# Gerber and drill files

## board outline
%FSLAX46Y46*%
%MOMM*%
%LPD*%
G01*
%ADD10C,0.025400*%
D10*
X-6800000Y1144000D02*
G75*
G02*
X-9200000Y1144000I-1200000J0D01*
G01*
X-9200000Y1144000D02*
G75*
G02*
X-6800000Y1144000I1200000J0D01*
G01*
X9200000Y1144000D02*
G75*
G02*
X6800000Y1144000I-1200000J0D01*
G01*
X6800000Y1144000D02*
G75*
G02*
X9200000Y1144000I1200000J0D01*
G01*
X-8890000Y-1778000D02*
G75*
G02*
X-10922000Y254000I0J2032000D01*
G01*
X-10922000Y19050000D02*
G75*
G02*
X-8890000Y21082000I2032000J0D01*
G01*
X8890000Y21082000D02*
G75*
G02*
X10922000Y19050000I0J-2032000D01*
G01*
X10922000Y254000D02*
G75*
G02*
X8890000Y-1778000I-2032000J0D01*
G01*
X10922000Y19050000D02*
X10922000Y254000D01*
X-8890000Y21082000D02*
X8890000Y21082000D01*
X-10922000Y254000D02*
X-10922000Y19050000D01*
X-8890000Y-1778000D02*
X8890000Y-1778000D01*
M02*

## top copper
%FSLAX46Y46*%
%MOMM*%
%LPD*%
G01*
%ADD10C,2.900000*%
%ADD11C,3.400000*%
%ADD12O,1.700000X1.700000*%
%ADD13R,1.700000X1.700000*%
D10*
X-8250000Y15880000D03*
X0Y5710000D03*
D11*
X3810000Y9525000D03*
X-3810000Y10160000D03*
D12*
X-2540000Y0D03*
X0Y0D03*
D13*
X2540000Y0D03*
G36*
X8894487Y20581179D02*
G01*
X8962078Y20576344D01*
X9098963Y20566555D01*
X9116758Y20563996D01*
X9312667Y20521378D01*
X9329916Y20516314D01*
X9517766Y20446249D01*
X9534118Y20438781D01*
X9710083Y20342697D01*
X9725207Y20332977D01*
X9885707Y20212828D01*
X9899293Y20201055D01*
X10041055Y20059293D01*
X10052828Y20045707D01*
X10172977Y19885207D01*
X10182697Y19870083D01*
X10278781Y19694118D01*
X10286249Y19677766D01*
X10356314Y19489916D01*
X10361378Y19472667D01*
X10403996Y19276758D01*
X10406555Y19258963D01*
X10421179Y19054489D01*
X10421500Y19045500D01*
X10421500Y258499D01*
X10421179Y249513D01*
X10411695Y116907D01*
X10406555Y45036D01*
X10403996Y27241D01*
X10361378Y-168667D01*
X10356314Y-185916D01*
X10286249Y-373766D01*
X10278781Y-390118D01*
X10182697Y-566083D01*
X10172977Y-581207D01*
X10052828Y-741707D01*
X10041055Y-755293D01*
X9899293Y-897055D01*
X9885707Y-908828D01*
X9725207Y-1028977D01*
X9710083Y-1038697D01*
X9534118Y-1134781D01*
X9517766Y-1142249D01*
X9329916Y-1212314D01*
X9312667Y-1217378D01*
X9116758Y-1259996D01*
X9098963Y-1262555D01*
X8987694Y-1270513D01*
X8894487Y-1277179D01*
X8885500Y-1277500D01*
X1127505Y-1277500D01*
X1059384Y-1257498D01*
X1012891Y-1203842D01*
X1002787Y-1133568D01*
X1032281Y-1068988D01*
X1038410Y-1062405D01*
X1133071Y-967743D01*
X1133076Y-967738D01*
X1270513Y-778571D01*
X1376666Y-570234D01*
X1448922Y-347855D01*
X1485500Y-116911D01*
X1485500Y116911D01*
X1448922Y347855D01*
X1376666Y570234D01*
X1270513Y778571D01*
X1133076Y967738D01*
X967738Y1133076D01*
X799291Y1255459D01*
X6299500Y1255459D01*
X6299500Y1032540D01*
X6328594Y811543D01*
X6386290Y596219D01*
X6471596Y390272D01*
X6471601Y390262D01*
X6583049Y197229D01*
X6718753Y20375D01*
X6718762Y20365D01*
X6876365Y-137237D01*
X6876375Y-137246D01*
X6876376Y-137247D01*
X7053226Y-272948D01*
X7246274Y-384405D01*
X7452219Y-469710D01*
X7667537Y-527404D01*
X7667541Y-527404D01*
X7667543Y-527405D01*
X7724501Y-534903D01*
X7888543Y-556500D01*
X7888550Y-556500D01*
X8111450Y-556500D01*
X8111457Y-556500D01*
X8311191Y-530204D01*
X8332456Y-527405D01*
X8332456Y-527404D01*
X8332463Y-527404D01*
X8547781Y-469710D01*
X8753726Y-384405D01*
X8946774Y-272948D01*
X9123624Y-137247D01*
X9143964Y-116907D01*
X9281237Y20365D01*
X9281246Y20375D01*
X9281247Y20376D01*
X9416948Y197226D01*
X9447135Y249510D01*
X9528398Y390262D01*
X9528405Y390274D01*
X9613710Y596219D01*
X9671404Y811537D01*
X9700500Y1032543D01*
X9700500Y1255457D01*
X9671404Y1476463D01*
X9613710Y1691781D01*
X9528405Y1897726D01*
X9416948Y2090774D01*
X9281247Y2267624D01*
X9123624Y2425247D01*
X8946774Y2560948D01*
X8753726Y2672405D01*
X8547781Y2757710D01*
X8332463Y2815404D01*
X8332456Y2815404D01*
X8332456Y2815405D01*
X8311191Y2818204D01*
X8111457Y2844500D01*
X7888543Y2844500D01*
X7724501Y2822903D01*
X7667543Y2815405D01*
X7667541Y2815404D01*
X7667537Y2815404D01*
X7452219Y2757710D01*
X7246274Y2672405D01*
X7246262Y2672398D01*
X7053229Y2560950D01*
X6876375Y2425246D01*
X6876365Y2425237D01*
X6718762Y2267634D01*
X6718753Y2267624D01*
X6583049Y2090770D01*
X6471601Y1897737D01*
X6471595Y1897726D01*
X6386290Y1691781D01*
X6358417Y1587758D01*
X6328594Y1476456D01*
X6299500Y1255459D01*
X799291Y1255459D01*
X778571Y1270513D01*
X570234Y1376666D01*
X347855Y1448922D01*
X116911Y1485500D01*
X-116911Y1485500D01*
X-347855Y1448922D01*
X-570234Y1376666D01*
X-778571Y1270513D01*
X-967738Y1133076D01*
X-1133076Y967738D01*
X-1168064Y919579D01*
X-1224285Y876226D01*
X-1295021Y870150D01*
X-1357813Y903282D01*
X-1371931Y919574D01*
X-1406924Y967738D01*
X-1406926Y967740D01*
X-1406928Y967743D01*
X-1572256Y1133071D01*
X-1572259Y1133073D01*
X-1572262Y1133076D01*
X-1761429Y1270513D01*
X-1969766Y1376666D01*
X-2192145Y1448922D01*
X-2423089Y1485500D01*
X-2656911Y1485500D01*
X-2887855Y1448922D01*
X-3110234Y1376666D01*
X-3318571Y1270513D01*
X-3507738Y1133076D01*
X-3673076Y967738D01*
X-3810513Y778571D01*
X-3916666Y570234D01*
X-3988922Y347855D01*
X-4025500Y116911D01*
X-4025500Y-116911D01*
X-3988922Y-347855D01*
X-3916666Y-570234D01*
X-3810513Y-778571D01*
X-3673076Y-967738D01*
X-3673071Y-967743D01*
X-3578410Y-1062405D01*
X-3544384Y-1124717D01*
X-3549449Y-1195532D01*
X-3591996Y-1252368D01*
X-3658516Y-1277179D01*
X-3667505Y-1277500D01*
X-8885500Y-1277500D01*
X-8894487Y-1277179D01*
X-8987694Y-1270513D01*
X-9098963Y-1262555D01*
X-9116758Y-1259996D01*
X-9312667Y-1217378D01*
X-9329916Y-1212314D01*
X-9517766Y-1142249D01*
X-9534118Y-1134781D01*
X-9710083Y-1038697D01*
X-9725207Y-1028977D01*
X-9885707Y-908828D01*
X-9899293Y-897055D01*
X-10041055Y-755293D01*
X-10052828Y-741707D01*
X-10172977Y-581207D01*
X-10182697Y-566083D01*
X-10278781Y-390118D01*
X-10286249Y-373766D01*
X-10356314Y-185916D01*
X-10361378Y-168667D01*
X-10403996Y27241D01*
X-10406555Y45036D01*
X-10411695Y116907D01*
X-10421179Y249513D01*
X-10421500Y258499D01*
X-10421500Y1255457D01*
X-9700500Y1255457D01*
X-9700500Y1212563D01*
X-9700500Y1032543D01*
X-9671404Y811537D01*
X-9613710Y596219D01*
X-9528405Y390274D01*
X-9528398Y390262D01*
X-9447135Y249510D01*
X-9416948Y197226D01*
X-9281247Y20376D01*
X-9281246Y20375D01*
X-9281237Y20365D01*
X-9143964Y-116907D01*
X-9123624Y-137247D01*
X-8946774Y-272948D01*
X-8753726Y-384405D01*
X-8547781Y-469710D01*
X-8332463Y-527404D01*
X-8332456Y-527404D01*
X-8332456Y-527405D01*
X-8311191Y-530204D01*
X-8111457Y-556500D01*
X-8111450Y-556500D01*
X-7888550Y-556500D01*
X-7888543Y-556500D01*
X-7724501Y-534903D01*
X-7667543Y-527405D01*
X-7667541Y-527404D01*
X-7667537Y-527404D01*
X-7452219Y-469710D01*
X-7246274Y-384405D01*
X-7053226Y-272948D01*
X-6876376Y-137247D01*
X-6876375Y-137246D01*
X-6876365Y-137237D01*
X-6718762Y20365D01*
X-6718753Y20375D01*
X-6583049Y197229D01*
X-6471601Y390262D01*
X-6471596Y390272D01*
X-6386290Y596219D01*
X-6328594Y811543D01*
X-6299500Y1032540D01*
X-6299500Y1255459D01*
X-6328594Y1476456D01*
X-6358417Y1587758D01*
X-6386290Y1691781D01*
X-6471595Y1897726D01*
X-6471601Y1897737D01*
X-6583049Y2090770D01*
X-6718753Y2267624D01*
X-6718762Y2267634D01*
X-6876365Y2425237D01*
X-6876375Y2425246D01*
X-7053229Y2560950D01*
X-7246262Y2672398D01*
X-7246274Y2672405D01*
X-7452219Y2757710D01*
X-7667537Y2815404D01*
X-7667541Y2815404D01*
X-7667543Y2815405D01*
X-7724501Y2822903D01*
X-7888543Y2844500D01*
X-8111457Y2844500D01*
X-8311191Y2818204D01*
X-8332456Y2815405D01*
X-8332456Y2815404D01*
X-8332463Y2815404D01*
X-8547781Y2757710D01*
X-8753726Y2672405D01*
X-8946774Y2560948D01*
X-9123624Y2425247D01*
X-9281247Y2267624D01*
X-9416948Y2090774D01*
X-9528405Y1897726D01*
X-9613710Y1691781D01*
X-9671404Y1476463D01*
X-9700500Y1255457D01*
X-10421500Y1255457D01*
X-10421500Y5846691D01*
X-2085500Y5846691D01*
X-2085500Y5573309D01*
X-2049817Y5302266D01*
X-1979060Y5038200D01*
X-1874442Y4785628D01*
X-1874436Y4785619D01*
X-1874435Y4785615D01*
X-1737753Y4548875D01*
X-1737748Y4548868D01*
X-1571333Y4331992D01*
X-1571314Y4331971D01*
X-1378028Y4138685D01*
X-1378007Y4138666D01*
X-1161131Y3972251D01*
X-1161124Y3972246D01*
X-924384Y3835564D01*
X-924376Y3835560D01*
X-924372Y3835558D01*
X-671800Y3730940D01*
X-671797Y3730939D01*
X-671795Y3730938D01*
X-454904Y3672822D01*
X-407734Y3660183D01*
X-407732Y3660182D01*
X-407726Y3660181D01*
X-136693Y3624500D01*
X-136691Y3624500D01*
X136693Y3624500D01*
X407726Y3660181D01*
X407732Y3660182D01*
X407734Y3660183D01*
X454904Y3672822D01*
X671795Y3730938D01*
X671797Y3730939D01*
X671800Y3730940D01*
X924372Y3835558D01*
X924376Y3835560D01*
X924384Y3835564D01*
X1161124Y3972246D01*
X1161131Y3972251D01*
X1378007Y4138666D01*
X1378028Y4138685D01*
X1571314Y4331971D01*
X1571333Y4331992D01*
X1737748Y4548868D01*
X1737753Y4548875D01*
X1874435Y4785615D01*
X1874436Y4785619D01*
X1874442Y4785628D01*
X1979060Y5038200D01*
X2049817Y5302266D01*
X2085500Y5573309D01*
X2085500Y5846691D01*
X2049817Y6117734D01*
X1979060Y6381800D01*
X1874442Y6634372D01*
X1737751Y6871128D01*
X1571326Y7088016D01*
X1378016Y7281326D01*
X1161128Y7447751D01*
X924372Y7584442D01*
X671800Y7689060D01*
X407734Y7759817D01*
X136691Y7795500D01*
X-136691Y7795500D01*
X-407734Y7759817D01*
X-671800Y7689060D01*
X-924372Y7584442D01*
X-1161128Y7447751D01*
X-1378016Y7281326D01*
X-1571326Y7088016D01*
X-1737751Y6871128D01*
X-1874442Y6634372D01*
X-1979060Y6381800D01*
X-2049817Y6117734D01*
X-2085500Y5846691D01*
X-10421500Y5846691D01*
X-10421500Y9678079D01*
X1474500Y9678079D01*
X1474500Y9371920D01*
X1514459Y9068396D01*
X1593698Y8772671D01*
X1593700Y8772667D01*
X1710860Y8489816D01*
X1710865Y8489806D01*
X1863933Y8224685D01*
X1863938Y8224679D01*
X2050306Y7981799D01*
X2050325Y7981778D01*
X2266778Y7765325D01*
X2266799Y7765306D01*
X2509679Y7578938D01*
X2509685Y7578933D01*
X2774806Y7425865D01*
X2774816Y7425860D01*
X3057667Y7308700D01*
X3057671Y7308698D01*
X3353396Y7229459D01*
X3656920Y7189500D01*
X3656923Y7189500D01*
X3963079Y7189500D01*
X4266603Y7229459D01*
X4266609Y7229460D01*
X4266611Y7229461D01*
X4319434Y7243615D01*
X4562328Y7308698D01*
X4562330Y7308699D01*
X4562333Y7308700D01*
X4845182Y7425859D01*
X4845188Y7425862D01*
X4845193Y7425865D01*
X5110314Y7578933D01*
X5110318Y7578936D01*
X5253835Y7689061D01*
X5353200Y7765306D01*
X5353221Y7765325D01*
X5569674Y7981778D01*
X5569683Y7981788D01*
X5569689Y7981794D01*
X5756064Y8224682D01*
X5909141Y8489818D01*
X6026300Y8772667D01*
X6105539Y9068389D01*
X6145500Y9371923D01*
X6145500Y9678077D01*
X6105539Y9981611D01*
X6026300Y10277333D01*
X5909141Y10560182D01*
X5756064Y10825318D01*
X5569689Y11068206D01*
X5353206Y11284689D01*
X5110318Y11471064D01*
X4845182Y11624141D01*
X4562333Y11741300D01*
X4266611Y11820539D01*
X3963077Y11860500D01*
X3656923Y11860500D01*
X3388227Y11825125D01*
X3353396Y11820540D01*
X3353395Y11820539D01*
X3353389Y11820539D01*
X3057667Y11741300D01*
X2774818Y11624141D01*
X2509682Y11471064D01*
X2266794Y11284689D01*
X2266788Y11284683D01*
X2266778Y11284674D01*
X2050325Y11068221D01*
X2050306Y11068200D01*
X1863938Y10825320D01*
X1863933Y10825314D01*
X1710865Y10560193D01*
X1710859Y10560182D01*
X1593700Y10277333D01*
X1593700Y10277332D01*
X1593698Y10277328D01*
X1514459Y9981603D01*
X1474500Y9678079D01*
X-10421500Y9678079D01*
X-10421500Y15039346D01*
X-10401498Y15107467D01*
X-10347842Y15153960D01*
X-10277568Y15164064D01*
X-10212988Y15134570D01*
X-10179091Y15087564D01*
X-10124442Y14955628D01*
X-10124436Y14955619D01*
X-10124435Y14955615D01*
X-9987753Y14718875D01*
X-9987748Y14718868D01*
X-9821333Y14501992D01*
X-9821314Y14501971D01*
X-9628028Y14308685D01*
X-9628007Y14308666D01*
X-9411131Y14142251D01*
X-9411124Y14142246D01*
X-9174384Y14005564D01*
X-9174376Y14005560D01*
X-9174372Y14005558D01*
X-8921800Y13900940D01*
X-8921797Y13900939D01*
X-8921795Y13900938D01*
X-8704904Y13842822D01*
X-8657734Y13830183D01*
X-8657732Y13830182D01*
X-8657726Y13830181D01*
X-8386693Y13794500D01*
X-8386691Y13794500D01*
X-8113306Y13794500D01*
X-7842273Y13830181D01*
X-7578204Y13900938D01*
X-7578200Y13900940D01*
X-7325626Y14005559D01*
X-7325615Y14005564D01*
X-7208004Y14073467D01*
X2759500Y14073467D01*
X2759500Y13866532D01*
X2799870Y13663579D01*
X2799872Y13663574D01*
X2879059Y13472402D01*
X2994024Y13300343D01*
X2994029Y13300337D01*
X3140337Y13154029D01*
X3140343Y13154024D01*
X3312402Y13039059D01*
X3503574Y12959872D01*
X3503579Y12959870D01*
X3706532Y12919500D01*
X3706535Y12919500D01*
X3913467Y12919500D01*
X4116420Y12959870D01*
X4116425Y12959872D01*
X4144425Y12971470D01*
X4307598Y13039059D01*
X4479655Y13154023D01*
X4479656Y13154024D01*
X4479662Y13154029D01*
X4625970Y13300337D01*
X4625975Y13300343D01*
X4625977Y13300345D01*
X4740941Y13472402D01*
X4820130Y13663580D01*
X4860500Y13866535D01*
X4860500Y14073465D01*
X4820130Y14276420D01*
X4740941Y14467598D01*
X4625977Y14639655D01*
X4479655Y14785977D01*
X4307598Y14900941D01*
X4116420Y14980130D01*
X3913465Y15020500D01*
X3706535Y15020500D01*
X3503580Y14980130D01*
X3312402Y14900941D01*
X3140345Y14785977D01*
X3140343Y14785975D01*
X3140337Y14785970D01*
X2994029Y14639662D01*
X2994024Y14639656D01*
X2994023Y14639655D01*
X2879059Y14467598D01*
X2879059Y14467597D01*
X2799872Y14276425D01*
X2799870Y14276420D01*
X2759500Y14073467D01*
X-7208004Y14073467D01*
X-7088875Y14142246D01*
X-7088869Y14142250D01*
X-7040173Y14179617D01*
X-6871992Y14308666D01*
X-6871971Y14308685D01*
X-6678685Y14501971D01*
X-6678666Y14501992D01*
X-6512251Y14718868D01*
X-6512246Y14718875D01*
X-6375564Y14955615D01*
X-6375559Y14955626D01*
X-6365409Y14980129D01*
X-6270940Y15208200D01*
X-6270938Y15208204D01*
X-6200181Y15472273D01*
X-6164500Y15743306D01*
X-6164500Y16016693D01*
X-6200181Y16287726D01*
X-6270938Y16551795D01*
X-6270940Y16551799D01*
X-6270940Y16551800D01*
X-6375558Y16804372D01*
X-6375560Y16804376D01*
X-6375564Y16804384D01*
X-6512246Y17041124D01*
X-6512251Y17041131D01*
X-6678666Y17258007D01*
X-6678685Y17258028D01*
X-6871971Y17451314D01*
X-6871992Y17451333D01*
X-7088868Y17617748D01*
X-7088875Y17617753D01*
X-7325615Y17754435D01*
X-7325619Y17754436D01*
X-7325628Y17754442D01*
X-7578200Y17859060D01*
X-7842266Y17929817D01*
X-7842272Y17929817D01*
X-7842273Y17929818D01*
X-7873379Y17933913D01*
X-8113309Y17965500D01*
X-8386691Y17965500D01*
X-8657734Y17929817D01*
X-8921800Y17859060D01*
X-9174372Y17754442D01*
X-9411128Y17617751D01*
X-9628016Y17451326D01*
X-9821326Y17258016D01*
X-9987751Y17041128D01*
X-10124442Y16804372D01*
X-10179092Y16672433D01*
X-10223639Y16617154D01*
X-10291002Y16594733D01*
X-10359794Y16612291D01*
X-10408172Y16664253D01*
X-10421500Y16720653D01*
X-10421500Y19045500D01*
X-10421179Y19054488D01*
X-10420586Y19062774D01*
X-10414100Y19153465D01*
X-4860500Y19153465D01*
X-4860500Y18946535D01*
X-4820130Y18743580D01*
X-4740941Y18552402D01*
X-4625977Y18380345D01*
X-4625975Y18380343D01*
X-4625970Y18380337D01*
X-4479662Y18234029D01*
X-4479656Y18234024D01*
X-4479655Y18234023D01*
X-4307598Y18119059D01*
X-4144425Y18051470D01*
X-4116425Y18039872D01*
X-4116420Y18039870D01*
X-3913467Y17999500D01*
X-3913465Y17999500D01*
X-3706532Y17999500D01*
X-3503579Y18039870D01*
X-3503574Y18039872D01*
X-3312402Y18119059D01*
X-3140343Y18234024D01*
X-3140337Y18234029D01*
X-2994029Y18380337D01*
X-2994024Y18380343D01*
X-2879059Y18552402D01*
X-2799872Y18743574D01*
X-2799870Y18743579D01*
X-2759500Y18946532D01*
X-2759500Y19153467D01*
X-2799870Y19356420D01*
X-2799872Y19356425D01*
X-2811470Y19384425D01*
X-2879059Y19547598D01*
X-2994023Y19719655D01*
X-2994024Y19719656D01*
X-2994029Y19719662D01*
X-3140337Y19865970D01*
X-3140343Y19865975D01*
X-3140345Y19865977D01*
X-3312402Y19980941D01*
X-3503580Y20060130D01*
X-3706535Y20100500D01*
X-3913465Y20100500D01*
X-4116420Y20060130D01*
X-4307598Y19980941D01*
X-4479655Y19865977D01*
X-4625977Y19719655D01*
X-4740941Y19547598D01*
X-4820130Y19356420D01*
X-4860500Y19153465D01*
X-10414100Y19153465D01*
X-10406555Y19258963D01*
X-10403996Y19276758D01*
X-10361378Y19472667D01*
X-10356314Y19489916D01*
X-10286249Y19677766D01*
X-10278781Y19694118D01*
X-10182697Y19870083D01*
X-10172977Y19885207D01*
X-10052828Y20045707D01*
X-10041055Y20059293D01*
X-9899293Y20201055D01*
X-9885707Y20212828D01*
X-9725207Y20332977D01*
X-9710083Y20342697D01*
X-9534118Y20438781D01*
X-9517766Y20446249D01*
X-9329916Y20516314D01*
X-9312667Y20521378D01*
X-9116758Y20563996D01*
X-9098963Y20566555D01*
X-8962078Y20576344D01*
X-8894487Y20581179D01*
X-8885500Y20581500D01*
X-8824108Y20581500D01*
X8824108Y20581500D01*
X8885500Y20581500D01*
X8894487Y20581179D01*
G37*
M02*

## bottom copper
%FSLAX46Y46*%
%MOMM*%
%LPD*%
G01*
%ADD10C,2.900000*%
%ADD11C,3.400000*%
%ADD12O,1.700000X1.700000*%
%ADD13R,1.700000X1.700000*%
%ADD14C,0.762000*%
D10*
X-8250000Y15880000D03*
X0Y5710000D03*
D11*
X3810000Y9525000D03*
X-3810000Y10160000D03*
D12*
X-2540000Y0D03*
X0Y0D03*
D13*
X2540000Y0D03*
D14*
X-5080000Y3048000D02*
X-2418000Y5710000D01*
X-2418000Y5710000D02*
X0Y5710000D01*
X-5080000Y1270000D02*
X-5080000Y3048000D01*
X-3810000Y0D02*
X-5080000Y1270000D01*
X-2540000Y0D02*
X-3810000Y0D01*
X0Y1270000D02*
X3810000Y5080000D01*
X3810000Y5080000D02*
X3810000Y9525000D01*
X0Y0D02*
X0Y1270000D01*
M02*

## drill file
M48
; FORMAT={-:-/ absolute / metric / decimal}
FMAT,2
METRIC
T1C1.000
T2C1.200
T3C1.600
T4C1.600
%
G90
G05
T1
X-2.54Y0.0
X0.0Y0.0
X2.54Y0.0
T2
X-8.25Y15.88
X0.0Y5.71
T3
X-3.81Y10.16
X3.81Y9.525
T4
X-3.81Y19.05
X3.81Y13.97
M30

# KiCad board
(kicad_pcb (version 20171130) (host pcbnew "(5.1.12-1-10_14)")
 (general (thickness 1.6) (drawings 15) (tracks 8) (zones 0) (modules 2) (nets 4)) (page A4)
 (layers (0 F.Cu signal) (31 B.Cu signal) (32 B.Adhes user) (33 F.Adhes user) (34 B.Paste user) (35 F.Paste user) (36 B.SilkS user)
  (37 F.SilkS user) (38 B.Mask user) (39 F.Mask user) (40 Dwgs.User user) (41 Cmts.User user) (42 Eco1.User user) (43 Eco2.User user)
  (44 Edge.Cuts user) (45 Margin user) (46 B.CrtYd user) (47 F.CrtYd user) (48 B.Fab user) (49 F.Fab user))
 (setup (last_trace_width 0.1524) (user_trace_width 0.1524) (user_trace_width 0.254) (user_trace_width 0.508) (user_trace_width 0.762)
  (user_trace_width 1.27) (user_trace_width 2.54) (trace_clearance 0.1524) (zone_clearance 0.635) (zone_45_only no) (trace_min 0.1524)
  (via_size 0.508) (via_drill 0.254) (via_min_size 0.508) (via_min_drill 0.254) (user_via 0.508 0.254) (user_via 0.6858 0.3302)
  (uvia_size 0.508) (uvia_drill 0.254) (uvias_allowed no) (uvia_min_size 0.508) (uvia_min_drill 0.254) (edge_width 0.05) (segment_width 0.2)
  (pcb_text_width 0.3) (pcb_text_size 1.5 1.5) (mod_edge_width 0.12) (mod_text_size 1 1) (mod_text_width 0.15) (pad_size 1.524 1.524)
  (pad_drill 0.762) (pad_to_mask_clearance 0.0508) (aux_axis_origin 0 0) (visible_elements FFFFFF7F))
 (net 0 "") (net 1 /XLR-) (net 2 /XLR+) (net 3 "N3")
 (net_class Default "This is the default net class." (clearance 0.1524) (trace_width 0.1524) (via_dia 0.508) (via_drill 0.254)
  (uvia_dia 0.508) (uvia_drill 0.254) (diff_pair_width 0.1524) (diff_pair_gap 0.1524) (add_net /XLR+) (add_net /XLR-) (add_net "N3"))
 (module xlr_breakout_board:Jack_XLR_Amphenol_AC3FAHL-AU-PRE (layer F.Cu) (at 0 -22.86)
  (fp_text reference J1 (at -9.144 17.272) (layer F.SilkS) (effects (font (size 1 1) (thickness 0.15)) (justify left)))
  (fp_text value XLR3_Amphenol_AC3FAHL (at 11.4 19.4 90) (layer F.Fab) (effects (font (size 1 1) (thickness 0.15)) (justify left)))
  (pad "" np_thru_hole circle (at 3.81 8.89) (size 1.6 1.6) (drill 1.6) (layers *.Cu *.Mask))
  (pad "" np_thru_hole circle (at -3.81 3.81) (size 1.6 1.6) (drill 1.6) (layers *.Cu *.Mask))
  (pad G thru_hole circle (at -8.25 6.98) (size 2.9 2.9) (drill 1.2) (layers *.Cu *.Mask))
  (pad 3 thru_hole circle (at 0 17.15) (size 2.9 2.9) (drill 1.2) (layers *.Cu *.Mask) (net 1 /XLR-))
  (pad 2 thru_hole circle (at 3.81 13.335) (size 3.4 3.4) (drill 1.6) (layers *.Cu *.Mask) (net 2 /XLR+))
  (pad 1 thru_hole circle (at -3.81 12.7) (size 3.4 3.4) (drill 1.6) (layers *.Cu *.Mask) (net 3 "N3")))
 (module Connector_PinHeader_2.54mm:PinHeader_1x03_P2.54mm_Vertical (layer F.Cu) (at 2.54 0 270)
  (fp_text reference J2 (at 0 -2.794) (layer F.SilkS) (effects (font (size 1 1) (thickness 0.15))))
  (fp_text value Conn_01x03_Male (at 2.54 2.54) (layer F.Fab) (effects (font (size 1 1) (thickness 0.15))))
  (pad 3 thru_hole oval (at 0 5.08 270) (size 1.7 1.7) (drill 1) (layers *.Cu *.Mask) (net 1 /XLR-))
  (pad 2 thru_hole oval (at 0 2.54 270) (size 1.7 1.7) (drill 1) (layers *.Cu *.Mask) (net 2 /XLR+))
  (pad 1 thru_hole rect (at 0 0 270) (size 1.7 1.7) (drill 1) (layers *.Cu *.Mask) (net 3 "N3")))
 (gr_circle (center -8 -1.144) (end -6.8 -1.144) (layer Edge.Cuts) (width 0.0254))
 (gr_circle (center 8 -1.144) (end 9.2 -1.144) (layer Edge.Cuts) (width 0.0254))
 (gr_arc (start -8.89 -0.254) (end -10.922 -0.254) (angle -90) (layer Edge.Cuts) (width 0.0254))
 (gr_arc (start -8.89 -19.05) (end -8.89 -21.082) (angle -90) (layer Edge.Cuts) (width 0.0254))
 (gr_arc (start 8.89 -19.05) (end 10.922 -19.05) (angle -90) (layer Edge.Cuts) (width 0.0254))
 (gr_arc (start 8.89 -0.254) (end 8.89 1.778) (angle -90) (layer Edge.Cuts) (width 0.0254))
 (gr_line (start 10.922 -19.05) (end 10.922 -0.254) (layer Edge.Cuts) (width 0.0254))
 (gr_line (start -8.89 -21.082) (end 8.89 -21.082) (layer Edge.Cuts) (width 0.0254))
 (gr_line (start -10.922 -0.254) (end -10.922 -19.05) (layer Edge.Cuts) (width 0.0254))
 (gr_line (start -8.89 1.778) (end 8.89 1.778) (layer Edge.Cuts) (width 0.0254))
 (segment (start -5.08 -3.048) (end -2.418 -5.71) (width 0.762) (layer B.Cu) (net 1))
 (segment (start -2.418 -5.71) (end 0 -5.71) (width 0.762) (layer B.Cu) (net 1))
 (segment (start -5.08 -1.27) (end -5.08 -3.048) (width 0.762) (layer B.Cu) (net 1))
 (segment (start -3.81 0) (end -5.08 -1.27) (width 0.762) (layer B.Cu) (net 1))
 (segment (start -2.54 0) (end -3.81 0) (width 0.762) (layer B.Cu) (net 1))
 (segment (start 0 -1.27) (end 3.81 -5.08) (width 0.762) (layer B.Cu) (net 2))
 (segment (start 3.81 -5.08) (end 3.81 -9.525) (width 0.762) (layer B.Cu) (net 2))
 (segment (start 0 0) (end 0 -1.27) (width 0.762) (layer B.Cu) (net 2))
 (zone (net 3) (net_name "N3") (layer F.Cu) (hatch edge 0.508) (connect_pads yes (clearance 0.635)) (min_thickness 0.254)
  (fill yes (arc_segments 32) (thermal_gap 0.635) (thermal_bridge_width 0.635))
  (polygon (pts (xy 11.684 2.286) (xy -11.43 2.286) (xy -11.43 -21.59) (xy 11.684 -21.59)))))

